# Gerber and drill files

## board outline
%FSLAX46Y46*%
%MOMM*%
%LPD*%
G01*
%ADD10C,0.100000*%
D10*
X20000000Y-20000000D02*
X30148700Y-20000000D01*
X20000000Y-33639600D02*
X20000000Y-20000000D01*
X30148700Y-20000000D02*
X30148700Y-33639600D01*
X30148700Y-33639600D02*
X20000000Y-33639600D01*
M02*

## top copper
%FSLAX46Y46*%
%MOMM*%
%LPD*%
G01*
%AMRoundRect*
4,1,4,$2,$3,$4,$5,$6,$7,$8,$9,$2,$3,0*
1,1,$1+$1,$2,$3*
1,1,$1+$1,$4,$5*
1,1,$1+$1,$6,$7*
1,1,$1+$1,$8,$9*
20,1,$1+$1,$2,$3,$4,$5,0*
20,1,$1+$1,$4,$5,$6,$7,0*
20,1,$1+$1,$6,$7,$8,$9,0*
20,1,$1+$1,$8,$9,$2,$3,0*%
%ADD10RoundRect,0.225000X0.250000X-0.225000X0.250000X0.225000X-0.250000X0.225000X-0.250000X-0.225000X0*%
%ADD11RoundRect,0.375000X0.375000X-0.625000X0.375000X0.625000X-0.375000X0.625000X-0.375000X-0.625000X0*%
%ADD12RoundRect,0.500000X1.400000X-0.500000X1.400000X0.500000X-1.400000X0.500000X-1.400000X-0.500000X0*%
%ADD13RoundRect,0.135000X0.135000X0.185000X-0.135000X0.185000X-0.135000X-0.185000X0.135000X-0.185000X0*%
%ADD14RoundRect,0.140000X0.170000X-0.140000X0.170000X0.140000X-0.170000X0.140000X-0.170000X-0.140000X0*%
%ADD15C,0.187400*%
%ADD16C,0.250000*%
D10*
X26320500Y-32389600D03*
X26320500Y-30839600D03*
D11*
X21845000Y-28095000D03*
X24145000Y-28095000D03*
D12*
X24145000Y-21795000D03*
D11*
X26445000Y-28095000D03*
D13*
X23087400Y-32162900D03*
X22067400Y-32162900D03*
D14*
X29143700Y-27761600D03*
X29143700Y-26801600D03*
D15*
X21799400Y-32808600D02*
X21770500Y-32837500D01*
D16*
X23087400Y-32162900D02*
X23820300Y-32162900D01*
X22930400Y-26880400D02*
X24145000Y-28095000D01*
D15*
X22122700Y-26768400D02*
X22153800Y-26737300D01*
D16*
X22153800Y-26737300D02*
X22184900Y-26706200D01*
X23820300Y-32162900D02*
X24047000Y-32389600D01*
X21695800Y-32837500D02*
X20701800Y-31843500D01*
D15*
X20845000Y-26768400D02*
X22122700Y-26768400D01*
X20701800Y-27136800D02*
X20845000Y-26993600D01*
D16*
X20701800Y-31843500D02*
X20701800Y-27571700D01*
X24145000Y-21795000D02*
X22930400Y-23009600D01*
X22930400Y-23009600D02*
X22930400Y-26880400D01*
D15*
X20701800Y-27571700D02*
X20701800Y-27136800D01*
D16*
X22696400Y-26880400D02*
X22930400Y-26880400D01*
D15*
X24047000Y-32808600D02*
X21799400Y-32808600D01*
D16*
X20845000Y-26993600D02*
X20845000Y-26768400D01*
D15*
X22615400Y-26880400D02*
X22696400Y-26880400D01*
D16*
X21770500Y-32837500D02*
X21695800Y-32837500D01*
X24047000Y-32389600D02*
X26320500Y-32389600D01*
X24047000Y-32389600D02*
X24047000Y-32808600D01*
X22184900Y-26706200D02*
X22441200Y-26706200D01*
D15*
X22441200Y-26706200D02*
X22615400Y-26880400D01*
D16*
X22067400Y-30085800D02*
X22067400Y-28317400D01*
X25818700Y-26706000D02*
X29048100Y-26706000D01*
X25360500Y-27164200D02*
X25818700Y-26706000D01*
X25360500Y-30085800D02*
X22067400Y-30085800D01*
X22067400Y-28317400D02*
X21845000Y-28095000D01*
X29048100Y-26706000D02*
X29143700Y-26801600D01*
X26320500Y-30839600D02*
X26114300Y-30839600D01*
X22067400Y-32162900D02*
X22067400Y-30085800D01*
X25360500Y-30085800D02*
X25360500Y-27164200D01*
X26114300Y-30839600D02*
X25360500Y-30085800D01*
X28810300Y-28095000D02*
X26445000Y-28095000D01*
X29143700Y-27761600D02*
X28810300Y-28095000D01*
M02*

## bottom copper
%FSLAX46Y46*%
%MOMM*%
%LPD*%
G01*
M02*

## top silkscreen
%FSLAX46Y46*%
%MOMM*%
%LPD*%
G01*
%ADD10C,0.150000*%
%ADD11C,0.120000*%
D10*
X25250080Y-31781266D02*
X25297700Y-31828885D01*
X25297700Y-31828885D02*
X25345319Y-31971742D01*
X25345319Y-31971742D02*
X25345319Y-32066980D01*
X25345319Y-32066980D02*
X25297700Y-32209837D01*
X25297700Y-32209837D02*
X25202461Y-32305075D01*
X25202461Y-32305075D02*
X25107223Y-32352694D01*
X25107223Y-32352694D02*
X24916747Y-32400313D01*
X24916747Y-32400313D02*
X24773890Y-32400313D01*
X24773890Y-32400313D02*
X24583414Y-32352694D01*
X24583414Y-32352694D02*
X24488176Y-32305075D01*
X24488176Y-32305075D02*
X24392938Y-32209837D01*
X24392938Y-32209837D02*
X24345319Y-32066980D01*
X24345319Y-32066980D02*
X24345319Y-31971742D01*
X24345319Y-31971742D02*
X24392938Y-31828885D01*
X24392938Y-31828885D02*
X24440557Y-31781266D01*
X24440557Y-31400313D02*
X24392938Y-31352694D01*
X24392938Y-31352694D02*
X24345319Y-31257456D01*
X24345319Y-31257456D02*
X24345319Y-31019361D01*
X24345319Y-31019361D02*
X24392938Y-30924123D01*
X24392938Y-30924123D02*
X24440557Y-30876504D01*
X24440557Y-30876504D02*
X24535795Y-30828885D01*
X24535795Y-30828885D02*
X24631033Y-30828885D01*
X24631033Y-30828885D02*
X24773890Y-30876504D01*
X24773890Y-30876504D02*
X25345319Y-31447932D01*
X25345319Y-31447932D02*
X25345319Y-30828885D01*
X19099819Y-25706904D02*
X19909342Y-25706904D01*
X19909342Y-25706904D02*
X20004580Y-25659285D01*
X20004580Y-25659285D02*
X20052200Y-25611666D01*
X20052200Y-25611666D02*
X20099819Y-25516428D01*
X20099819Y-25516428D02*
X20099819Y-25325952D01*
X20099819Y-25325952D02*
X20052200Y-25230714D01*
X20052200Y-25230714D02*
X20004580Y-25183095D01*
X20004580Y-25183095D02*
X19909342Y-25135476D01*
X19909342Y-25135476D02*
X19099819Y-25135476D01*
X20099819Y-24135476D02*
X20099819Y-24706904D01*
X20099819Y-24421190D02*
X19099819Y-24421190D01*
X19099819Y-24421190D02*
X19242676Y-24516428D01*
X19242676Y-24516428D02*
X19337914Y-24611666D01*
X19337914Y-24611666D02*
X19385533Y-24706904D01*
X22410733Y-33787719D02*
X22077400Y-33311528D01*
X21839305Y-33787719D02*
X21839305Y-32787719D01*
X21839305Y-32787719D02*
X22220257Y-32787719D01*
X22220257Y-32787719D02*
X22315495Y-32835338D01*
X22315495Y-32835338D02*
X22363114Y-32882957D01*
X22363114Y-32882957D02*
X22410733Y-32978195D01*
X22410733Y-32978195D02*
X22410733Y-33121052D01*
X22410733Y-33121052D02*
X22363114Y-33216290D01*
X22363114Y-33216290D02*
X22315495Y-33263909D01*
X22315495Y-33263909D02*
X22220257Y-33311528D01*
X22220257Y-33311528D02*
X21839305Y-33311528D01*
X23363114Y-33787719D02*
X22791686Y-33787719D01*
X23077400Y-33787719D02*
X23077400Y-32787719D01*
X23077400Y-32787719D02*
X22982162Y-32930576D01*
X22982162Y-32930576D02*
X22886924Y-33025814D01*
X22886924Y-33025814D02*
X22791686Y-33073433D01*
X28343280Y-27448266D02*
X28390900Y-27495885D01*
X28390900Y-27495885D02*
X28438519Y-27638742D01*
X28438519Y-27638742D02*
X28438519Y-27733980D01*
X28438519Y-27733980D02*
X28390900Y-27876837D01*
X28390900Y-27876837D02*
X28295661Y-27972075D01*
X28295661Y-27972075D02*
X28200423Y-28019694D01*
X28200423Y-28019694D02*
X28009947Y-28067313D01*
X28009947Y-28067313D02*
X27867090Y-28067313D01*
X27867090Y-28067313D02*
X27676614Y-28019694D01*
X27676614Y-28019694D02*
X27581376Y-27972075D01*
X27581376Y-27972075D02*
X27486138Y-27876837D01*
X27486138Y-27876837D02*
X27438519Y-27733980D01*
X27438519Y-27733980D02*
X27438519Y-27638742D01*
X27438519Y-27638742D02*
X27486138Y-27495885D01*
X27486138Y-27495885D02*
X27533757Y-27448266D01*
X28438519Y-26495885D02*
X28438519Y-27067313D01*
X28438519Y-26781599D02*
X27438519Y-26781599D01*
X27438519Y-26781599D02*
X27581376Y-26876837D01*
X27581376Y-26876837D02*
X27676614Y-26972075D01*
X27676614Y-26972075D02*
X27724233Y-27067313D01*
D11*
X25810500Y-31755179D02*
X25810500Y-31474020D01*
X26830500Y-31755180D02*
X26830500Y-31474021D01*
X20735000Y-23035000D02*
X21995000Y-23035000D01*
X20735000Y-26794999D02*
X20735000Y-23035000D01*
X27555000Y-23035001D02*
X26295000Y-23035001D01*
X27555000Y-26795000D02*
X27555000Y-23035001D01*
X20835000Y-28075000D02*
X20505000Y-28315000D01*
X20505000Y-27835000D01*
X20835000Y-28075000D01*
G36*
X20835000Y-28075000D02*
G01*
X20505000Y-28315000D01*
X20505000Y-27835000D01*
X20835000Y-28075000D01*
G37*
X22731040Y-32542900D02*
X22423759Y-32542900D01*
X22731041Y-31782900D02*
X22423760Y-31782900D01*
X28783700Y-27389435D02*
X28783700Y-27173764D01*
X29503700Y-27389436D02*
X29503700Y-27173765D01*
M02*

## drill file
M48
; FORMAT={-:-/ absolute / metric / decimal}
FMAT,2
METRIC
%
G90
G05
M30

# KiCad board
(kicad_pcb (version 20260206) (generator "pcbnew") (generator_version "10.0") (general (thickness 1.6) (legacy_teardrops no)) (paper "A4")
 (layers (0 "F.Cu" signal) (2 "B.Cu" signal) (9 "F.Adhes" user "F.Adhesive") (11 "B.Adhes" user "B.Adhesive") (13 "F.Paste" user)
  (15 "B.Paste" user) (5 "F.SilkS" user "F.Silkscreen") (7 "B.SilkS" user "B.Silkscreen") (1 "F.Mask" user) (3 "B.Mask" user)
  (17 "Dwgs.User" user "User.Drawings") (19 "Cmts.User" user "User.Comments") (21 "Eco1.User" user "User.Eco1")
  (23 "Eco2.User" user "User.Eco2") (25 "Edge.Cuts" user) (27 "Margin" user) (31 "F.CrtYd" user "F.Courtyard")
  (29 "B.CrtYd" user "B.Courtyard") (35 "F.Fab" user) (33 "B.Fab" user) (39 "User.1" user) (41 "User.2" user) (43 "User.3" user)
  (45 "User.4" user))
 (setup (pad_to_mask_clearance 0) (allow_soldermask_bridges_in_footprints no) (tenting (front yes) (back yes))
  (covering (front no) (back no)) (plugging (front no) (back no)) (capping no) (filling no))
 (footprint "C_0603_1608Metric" (layer "F.Cu") (at 26.3205 31.6146 90)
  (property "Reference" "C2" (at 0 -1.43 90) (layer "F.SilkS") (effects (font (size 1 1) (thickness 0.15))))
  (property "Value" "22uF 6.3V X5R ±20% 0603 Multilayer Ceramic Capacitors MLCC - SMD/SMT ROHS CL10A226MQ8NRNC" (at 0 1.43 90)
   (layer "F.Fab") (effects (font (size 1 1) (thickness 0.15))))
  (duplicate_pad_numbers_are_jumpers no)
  (fp_line (start -0.140579 -0.51) (end 0.14058 -0.51) (stroke (width 0.12) (type solid)) (layer "F.SilkS"))
  (fp_line (start -0.14058 0.51) (end 0.140579 0.51) (stroke (width 0.12) (type solid)) (layer "F.SilkS"))
  (pad "1" smd roundrect (at -0.775 0 90) (size 0.9 0.95) (layers "F.Cu" "F.Mask" "F.Paste") (roundrect_rratio 0.25) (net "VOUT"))
  (pad "2" smd roundrect (at 0.775 0 90) (size 0.9 0.95) (layers "F.Cu" "F.Mask" "F.Paste") (roundrect_rratio 0.25) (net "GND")))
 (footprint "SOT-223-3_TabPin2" (layer "F.Cu") (at 24.145 24.945 90)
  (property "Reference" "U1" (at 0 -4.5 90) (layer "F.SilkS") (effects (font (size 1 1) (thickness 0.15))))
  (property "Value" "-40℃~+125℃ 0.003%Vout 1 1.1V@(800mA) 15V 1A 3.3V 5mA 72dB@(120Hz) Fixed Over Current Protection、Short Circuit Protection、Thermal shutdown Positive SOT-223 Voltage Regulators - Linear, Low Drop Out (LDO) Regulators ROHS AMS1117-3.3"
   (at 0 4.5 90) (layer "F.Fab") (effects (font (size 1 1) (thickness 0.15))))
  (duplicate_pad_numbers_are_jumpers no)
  (fp_line (start 1.91 -3.41) (end 1.91 -2.15) (stroke (width 0.12) (type solid)) (layer "F.SilkS"))
  (fp_line (start -1.849999 -3.41) (end 1.91 -3.41) (stroke (width 0.12) (type solid)) (layer "F.SilkS"))
  (fp_line (start 1.909999 3.41) (end 1.909999 2.15) (stroke (width 0.12) (type solid)) (layer "F.SilkS"))
  (fp_line (start -1.85 3.41) (end 1.909999 3.41) (stroke (width 0.12) (type solid)) (layer "F.SilkS"))
  (fp_poly (pts (xy -3.13 -3.31) (xy -3.37 -3.64) (xy -2.89 -3.64)) (stroke (width 0.12) (type solid)) (fill yes) (layer "F.SilkS"))
  (pad "1" smd roundrect (at -3.15 -2.3 90) (size 2 1.5) (layers "F.Cu" "F.Mask" "F.Paste") (roundrect_rratio 0.25) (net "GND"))
  (pad "2" smd roundrect (at -3.15 0 90) (size 2 1.5) (layers "F.Cu" "F.Mask" "F.Paste") (roundrect_rratio 0.25) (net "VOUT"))
  (pad "2" smd roundrect (at 3.15 0 90) (size 2 3.8) (layers "F.Cu" "F.Mask" "F.Paste") (roundrect_rratio 0.25) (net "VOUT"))
  (pad "3" smd roundrect (at -3.15 2.3 90) (size 2 1.5) (layers "F.Cu" "F.Mask" "F.Paste") (roundrect_rratio 0.25) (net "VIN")))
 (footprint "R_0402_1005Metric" (layer "F.Cu") (at 22.5774 32.1629 180)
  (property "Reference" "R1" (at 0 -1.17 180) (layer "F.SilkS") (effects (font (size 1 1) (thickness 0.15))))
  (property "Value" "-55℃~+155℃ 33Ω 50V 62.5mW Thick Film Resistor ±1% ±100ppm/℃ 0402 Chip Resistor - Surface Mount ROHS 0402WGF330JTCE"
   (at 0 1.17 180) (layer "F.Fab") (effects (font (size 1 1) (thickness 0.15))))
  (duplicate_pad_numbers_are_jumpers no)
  (fp_line (start -0.15364 -0.38) (end 0.153641 -0.38) (stroke (width 0.12) (type solid)) (layer "F.SilkS"))
  (fp_line (start -0.153641 0.38) (end 0.15364 0.38) (stroke (width 0.12) (type solid)) (layer "F.SilkS"))
  (pad "1" smd roundrect (at -0.51 0 180) (size 0.54 0.64) (layers "F.Cu" "F.Mask" "F.Paste") (roundrect_rratio 0.25) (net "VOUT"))
  (pad "2" smd roundrect (at 0.51 0 180) (size 0.54 0.64) (layers "F.Cu" "F.Mask" "F.Paste") (roundrect_rratio 0.25) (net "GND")))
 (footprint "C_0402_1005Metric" (layer "F.Cu") (at 29.1437 27.2816 90)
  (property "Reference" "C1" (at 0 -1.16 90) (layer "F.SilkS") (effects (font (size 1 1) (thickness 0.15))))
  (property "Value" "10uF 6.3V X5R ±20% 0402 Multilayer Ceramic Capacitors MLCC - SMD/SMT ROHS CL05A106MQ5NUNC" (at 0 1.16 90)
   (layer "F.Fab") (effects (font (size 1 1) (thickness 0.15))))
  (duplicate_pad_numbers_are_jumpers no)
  (fp_line (start -0.107835 -0.36) (end 0.107836 -0.36) (stroke (width 0.12) (type solid)) (layer "F.SilkS"))
  (fp_line (start -0.107836 0.36) (end 0.107835 0.36) (stroke (width 0.12) (type solid)) (layer "F.SilkS"))
  (pad "1" smd roundrect (at -0.48 0 90) (size 0.56 0.62) (layers "F.Cu" "F.Mask" "F.Paste") (roundrect_rratio 0.25) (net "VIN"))
  (pad "2" smd roundrect (at 0.48 0 90) (size 0.56 0.62) (layers "F.Cu" "F.Mask" "F.Paste") (roundrect_rratio 0.25) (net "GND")))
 (gr_line (start 20 20) (end 30.1487 20) (stroke (width 0.1) (type default)) (layer "Edge.Cuts"))
 (gr_line (start 20 33.6396) (end 20 20) (stroke (width 0.1) (type default)) (layer "Edge.Cuts"))
 (gr_line (start 30.1487 20) (end 30.1487 33.6396) (stroke (width 0.1) (type default)) (layer "Edge.Cuts"))
 (gr_line (start 30.1487 33.6396) (end 20 33.6396) (stroke (width 0.1) (type default)) (layer "Edge.Cuts"))
 (segment (start 21.7994 32.8086) (end 21.7705 32.8375) (width 0.1874) (layer "F.Cu") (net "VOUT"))
 (segment (start 23.0874 32.1629) (end 23.8203 32.1629) (width 0.25) (layer "F.Cu") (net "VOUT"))
 (segment (start 22.9304 26.8804) (end 24.145 28.095) (width 0.25) (layer "F.Cu") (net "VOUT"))
 (segment (start 22.1227 26.7684) (end 22.1538 26.7373) (width 0.1874) (layer "F.Cu") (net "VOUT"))
 (segment (start 22.1538 26.7373) (end 22.1849 26.7062) (width 0.25) (layer "F.Cu") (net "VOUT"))
 (segment (start 23.8203 32.1629) (end 24.047 32.3896) (width 0.25) (layer "F.Cu") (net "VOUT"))
 (segment (start 21.6958 32.8375) (end 20.7018 31.8435) (width 0.25) (layer "F.Cu") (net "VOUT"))
 (segment (start 20.845 26.7684) (end 22.1227 26.7684) (width 0.1874) (layer "F.Cu") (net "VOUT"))
 (segment (start 20.7018 27.1368) (end 20.845 26.9936) (width 0.1874) (layer "F.Cu") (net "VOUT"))
 (segment (start 20.7018 31.8435) (end 20.7018 27.5717) (width 0.25) (layer "F.Cu") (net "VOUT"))
 (segment (start 24.145 21.795) (end 22.9304 23.0096) (width 0.25) (layer "F.Cu") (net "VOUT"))
 (segment (start 22.9304 23.0096) (end 22.9304 26.8804) (width 0.25) (layer "F.Cu") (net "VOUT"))
 (segment (start 20.7018 27.5717) (end 20.7018 27.1368) (width 0.1874) (layer "F.Cu") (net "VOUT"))
 (segment (start 22.6964 26.8804) (end 22.9304 26.8804) (width 0.25) (layer "F.Cu") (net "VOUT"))
 (segment (start 24.047 32.8086) (end 21.7994 32.8086) (width 0.1874) (layer "F.Cu") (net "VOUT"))
 (segment (start 20.845 26.9936) (end 20.845 26.7684) (width 0.25) (layer "F.Cu") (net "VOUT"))
 (segment (start 22.6154 26.8804) (end 22.6964 26.8804) (width 0.1874) (layer "F.Cu") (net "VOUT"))
 (segment (start 21.7705 32.8375) (end 21.6958 32.8375) (width 0.25) (layer "F.Cu") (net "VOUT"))
 (segment (start 24.047 32.3896) (end 26.3205 32.3896) (width 0.25) (layer "F.Cu") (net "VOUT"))
 (segment (start 24.047 32.3896) (end 24.047 32.8086) (width 0.25) (layer "F.Cu") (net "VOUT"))
 (segment (start 22.1849 26.7062) (end 22.4412 26.7062) (width 0.25) (layer "F.Cu") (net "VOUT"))
 (segment (start 22.4412 26.7062) (end 22.6154 26.8804) (width 0.1874) (layer "F.Cu") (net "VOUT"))
 (segment (start 22.0674 30.0858) (end 22.0674 28.3174) (width 0.25) (layer "F.Cu") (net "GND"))
 (segment (start 25.8187 26.706) (end 29.0481 26.706) (width 0.25) (layer "F.Cu") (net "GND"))
 (segment (start 25.3605 27.1642) (end 25.8187 26.706) (width 0.25) (layer "F.Cu") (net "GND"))
 (segment (start 25.3605 30.0858) (end 22.0674 30.0858) (width 0.25) (layer "F.Cu") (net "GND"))
 (segment (start 22.0674 28.3174) (end 21.845 28.095) (width 0.25) (layer "F.Cu") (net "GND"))
 (segment (start 29.0481 26.706) (end 29.1437 26.8016) (width 0.25) (layer "F.Cu") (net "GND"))
 (segment (start 26.3205 30.8396) (end 26.1143 30.8396) (width 0.25) (layer "F.Cu") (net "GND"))
 (segment (start 22.0674 32.1629) (end 22.0674 30.0858) (width 0.25) (layer "F.Cu") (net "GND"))
 (segment (start 25.3605 30.0858) (end 25.3605 27.1642) (width 0.25) (layer "F.Cu") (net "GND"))
 (segment (start 26.1143 30.8396) (end 25.3605 30.0858) (width 0.25) (layer "F.Cu") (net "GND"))
 (segment (start 28.8103 28.095) (end 26.445 28.095) (width 0.25) (layer "F.Cu") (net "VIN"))
 (segment (start 29.1437 27.7616) (end 28.8103 28.095) (width 0.25) (layer "F.Cu") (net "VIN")))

